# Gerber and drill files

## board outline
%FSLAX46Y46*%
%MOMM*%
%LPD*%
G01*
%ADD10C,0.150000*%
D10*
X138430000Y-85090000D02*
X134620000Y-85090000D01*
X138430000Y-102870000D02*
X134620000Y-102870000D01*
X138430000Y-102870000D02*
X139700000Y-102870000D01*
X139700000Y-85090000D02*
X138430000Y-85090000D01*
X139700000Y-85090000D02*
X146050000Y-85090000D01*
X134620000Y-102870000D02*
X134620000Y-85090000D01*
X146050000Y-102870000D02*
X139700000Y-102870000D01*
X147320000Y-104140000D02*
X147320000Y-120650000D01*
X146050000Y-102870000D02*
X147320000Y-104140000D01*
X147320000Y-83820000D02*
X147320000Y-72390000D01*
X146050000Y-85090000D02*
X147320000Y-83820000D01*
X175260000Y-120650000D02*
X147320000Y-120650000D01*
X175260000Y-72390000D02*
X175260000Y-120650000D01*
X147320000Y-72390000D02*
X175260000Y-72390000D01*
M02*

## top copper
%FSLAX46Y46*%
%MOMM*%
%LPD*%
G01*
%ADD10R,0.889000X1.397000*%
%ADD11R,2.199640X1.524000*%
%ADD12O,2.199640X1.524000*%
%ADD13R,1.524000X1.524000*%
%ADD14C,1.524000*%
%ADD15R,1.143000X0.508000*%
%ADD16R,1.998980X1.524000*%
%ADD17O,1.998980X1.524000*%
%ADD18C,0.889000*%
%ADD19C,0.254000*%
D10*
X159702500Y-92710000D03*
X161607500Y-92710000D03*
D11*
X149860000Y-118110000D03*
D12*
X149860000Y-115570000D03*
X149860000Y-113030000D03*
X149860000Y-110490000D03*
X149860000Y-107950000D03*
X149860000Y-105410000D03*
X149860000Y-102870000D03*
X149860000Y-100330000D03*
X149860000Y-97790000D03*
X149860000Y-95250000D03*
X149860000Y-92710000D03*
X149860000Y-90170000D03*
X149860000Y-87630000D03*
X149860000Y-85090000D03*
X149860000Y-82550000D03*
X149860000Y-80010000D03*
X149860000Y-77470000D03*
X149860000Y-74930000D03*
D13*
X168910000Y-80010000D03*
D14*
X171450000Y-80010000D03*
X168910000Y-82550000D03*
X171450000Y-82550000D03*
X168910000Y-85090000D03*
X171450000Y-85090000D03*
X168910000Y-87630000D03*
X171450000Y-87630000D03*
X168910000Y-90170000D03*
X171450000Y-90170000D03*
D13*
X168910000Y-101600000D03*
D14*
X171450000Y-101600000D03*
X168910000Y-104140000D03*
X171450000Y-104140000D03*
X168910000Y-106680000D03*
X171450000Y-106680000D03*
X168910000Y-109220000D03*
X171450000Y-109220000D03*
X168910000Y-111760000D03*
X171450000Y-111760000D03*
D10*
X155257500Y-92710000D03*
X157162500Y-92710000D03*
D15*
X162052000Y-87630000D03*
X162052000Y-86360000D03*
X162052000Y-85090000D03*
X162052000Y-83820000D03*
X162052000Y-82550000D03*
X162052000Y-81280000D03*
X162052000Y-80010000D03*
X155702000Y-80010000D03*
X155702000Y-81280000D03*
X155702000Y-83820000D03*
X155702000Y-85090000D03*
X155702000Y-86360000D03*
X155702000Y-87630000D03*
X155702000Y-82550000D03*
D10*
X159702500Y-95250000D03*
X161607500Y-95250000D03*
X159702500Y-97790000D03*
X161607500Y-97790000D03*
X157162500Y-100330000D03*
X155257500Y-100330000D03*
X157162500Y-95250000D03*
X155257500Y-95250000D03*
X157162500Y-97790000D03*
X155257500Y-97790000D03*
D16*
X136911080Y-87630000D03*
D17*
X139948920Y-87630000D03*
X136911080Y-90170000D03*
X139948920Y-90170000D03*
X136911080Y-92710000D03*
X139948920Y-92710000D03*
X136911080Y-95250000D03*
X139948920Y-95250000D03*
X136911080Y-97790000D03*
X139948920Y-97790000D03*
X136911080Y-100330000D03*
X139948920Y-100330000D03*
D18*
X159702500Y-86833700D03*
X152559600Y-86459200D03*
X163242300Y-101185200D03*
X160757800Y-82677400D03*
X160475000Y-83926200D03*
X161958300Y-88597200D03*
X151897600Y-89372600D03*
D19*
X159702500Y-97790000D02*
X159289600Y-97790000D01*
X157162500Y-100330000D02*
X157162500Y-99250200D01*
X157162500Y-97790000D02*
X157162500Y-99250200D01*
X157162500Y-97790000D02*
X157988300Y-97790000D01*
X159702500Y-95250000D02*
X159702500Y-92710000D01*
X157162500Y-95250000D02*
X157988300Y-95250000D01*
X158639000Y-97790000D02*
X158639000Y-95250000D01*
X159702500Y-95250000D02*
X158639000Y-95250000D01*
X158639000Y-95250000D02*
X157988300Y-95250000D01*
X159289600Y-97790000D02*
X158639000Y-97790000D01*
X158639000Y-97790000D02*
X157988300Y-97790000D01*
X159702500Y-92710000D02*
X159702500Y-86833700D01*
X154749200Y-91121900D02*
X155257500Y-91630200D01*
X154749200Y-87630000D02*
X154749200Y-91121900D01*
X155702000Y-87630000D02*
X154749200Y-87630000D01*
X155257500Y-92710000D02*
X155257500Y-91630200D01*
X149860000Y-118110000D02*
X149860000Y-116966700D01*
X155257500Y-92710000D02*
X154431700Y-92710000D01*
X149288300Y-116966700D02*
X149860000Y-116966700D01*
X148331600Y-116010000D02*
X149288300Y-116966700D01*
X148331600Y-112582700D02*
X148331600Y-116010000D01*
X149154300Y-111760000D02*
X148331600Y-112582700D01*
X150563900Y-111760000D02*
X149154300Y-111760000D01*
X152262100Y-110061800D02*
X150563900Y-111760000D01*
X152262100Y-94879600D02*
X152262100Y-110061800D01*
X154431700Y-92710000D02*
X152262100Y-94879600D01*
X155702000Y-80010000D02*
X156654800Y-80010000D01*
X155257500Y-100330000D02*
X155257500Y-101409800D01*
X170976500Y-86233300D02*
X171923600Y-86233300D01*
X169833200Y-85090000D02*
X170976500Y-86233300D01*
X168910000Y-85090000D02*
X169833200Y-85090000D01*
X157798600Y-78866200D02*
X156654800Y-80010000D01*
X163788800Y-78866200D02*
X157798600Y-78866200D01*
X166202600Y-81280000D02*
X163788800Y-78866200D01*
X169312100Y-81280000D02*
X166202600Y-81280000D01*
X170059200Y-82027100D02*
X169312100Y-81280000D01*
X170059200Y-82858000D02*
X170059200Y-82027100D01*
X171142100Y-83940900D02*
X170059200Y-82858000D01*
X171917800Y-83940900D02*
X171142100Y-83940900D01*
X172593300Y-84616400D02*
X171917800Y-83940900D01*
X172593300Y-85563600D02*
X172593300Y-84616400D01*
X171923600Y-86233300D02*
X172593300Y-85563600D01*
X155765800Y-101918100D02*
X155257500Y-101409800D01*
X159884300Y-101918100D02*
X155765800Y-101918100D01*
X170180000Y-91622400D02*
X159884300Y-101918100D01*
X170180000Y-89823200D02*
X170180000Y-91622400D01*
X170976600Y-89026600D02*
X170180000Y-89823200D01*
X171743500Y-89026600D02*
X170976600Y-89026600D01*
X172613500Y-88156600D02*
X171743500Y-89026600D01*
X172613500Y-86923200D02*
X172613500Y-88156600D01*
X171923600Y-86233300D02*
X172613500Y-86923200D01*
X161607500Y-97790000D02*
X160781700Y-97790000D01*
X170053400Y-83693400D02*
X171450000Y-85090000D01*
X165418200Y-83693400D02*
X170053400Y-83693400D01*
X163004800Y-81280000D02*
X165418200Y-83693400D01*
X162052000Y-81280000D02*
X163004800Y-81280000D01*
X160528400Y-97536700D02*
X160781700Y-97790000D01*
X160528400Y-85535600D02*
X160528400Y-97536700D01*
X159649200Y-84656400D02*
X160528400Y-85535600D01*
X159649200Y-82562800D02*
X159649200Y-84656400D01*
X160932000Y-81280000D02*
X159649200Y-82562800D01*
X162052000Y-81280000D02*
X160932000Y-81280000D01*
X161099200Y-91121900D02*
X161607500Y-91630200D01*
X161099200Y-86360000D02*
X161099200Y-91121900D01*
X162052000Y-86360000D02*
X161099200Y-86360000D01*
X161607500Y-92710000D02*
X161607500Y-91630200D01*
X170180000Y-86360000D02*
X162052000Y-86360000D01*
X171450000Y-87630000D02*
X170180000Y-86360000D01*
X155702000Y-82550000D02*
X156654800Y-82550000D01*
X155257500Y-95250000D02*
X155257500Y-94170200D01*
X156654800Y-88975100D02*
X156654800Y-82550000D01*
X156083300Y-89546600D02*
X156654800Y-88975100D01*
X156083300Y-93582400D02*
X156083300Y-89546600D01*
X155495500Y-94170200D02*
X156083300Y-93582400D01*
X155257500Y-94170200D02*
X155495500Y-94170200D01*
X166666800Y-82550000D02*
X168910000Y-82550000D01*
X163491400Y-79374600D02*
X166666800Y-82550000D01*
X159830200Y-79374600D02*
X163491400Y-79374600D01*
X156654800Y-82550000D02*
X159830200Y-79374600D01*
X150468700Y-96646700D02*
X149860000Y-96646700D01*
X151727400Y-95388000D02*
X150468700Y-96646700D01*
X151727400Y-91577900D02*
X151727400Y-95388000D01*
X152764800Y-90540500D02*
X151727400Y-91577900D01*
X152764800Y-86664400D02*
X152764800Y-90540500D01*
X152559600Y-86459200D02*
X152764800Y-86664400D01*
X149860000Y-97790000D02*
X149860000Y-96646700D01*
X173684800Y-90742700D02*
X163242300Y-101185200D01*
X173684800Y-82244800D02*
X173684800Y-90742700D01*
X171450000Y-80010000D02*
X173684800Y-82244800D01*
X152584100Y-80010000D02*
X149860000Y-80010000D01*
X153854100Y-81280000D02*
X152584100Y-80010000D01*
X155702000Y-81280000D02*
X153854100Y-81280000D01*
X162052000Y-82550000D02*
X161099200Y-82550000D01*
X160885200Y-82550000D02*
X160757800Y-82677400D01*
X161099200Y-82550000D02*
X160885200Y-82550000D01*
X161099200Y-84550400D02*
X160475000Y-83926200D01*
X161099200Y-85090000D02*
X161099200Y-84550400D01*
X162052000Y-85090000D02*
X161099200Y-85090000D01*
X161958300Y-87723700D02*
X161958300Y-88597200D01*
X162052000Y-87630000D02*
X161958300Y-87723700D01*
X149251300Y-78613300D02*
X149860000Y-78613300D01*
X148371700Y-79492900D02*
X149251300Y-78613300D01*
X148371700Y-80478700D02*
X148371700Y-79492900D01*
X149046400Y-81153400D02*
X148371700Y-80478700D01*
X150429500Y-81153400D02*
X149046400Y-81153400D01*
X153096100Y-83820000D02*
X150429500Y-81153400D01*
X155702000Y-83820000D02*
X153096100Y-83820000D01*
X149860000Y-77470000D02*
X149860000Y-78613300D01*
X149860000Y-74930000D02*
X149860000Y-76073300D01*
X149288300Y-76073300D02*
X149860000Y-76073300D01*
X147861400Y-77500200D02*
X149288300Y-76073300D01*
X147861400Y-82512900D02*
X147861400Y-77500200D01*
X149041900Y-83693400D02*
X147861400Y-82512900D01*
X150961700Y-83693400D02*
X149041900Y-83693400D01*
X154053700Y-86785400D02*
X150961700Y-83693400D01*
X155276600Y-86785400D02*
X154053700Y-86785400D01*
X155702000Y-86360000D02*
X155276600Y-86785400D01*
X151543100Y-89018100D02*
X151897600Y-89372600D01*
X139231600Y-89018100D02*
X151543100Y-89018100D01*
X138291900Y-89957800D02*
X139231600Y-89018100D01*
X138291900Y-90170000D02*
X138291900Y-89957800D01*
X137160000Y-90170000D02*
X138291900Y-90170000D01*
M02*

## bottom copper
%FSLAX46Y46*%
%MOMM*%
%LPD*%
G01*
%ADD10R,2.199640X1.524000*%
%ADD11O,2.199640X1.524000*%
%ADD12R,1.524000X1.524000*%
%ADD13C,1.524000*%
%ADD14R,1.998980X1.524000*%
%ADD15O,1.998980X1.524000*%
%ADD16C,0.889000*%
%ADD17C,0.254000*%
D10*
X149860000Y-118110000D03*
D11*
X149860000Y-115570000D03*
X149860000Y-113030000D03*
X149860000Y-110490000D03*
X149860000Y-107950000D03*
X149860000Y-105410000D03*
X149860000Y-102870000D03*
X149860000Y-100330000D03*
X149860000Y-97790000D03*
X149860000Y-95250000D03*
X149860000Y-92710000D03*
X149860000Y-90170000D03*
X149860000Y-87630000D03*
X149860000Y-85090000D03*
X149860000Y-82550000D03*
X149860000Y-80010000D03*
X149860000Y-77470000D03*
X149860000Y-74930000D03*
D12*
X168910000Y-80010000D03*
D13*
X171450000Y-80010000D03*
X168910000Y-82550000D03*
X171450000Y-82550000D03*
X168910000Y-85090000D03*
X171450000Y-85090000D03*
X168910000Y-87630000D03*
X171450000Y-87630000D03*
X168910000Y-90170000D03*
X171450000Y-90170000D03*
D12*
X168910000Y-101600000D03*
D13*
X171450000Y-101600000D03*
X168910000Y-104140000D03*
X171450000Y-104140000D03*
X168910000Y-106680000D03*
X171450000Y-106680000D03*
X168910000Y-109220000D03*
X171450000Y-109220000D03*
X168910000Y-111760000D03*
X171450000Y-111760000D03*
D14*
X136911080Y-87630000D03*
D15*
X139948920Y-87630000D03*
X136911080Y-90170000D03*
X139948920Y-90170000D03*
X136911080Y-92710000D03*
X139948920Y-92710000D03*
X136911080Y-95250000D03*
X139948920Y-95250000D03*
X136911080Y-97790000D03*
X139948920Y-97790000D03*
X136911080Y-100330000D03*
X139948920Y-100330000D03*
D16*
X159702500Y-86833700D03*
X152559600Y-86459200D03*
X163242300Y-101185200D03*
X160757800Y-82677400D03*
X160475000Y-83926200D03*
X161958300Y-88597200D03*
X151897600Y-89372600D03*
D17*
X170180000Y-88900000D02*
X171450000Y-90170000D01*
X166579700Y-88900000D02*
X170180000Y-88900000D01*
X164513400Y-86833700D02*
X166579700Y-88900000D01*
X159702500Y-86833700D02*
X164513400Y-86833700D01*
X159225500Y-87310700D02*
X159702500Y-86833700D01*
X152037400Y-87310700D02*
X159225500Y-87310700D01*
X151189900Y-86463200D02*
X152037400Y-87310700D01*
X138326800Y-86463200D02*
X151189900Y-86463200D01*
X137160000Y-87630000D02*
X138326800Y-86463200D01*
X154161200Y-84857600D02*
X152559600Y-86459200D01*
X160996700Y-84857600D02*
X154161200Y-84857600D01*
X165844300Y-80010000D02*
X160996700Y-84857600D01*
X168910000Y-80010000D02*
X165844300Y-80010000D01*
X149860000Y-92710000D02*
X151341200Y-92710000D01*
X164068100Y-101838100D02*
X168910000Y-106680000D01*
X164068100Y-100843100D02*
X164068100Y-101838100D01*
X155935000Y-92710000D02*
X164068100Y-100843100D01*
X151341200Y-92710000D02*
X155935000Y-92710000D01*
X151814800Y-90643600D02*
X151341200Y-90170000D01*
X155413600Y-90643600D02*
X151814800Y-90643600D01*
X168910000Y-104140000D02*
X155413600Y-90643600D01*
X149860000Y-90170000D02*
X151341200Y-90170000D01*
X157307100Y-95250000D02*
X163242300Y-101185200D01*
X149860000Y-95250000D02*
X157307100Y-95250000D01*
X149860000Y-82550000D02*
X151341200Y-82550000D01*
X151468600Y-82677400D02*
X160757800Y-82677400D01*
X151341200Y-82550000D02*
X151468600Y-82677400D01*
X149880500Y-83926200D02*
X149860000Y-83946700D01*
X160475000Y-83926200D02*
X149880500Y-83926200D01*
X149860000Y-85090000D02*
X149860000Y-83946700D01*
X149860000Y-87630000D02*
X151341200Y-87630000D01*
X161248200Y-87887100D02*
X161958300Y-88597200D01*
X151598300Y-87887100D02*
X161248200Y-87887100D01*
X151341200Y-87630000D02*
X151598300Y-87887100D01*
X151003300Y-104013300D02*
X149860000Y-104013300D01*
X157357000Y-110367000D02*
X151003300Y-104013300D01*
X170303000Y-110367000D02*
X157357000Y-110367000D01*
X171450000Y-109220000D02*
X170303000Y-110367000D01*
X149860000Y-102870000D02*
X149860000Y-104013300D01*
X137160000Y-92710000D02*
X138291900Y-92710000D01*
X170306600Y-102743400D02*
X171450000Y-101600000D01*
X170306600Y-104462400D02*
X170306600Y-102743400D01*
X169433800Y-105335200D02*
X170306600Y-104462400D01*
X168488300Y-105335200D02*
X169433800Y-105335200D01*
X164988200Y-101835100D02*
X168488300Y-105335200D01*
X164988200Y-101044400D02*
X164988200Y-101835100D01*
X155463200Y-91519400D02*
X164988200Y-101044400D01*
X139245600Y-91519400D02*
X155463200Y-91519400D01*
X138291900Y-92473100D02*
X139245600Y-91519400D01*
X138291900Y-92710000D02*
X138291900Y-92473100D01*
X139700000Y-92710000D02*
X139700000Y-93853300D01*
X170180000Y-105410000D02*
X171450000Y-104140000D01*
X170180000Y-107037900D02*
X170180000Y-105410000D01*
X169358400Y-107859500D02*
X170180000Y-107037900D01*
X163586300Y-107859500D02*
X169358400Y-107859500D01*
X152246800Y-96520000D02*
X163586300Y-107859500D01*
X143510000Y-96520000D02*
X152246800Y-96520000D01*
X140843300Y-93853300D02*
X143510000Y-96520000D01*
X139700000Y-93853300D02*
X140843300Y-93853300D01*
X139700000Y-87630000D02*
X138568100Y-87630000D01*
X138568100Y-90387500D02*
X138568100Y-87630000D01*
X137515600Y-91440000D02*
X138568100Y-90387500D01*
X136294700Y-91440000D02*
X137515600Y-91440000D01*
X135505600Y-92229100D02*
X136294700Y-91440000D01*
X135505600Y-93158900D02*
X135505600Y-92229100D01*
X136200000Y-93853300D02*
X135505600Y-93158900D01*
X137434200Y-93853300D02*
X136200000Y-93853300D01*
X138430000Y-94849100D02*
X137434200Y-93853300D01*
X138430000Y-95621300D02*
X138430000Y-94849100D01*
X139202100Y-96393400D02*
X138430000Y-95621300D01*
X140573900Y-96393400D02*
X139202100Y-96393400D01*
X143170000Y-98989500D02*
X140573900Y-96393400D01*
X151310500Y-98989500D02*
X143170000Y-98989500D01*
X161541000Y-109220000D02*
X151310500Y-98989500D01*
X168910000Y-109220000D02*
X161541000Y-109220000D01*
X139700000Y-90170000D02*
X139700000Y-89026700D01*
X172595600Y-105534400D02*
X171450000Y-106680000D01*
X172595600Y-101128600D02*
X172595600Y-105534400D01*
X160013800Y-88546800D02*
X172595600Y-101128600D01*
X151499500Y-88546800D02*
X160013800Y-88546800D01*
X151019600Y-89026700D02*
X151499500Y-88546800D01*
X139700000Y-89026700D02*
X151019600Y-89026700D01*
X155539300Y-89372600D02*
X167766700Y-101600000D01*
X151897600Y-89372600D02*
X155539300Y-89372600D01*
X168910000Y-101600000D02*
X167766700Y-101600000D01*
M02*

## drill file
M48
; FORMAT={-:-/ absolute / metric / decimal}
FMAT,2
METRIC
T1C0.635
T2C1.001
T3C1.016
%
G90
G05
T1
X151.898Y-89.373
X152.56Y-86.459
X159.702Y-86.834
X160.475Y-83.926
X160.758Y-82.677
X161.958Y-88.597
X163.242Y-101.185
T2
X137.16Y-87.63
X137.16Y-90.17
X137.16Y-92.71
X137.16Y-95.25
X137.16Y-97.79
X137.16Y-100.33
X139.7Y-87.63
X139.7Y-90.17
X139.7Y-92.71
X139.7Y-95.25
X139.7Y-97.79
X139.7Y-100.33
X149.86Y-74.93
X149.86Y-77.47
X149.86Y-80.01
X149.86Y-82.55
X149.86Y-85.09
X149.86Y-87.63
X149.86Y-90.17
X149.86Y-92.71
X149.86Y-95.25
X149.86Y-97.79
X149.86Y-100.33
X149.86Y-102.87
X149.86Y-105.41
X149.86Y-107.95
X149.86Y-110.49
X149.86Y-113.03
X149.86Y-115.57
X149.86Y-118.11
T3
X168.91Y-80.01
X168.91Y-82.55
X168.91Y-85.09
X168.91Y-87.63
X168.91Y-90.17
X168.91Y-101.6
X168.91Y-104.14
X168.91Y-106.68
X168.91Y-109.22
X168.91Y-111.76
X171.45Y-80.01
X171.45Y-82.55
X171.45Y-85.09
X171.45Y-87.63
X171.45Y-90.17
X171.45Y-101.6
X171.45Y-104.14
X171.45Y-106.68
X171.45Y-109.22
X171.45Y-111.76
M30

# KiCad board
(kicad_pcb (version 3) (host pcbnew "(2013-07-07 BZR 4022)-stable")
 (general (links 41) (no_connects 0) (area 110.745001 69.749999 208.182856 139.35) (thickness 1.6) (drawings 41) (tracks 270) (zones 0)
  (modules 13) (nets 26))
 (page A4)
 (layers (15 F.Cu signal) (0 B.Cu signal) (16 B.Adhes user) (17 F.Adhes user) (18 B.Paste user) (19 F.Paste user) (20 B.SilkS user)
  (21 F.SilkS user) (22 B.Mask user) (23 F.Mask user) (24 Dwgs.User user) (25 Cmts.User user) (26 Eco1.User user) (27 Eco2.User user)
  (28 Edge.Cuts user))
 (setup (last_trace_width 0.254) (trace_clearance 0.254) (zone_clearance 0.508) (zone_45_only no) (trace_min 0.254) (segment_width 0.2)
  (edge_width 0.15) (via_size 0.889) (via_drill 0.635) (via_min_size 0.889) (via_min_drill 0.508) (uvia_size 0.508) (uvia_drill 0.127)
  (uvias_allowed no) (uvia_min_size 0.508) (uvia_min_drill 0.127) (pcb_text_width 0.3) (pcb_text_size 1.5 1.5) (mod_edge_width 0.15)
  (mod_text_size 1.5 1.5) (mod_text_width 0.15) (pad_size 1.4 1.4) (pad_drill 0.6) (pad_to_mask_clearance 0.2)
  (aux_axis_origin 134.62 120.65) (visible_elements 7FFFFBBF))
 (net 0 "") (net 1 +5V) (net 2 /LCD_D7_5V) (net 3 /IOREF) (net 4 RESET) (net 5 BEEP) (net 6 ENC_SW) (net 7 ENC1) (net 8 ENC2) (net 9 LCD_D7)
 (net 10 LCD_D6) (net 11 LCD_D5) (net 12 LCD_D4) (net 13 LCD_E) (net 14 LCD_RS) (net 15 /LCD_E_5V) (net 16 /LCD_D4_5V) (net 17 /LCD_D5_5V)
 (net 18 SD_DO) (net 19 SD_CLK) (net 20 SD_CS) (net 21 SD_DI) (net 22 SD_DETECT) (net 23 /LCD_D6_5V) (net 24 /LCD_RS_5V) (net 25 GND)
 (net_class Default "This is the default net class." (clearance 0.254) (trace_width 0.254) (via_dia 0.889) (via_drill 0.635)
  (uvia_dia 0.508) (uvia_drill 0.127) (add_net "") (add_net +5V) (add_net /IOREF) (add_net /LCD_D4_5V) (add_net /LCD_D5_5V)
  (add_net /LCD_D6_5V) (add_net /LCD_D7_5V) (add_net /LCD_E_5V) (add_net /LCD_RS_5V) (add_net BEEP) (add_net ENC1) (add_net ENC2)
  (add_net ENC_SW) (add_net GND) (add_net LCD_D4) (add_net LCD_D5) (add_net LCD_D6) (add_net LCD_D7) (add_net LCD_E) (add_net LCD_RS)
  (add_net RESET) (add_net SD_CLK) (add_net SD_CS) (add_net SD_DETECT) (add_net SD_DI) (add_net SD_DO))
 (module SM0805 (layer F.Cu) (at 160.655 92.71)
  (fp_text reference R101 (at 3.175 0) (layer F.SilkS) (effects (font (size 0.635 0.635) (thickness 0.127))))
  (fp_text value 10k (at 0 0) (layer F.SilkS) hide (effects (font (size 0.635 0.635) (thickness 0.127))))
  (pad 1 smd rect (at -0.9525 0) (size 0.889 1.397) (layers F.Cu F.Paste F.Mask) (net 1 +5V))
  (pad 2 smd rect (at 0.9525 0) (size 0.889 1.397) (layers F.Cu F.Paste F.Mask) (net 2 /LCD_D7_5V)))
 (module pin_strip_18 (layer B.Cu) (at 149.86 96.52 90)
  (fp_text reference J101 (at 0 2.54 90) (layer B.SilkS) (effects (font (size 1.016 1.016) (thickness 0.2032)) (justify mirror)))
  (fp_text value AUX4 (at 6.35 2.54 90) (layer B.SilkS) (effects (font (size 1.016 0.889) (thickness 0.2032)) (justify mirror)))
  (pad 1 thru_hole rect (at -21.59 0 90) (size 1.524 2.19964) (drill 1.00076) (layers *.Cu *.Mask B.SilkS) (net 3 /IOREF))
  (pad 2 thru_hole oval (at -19.05 0 90) (size 1.524 2.19964) (drill 1.00076) (layers *.Cu *.Mask B.SilkS))
  (pad 3 thru_hole oval (at -16.51 0 90) (size 1.524 2.19964) (drill 1.00076) (layers *.Cu *.Mask B.SilkS))
  (pad 4 thru_hole oval (at -13.97 0 90) (size 1.524 2.19964) (drill 1.00076) (layers *.Cu *.Mask B.SilkS))
  (pad 5 thru_hole oval (at -11.43 0 90) (size 1.524 2.19964) (drill 1.00076) (layers *.Cu *.Mask B.SilkS))
  (pad 6 thru_hole oval (at -8.89 0 90) (size 1.524 2.19964) (drill 1.00076) (layers *.Cu *.Mask B.SilkS))
  (pad 7 thru_hole oval (at -6.35 0 90) (size 1.524 2.19964) (drill 1.00076) (layers *.Cu *.Mask B.SilkS) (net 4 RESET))
  (pad 8 thru_hole oval (at -3.81 0 90) (size 1.524 2.19964) (drill 1.00076) (layers *.Cu *.Mask B.SilkS))
  (pad 9 thru_hole oval (at -1.27 0 90) (size 1.524 2.19964) (drill 1.00076) (layers *.Cu *.Mask B.SilkS) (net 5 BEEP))
  (pad 10 thru_hole oval (at 1.27 0 90) (size 1.524 2.19964) (drill 1.00076) (layers *.Cu *.Mask B.SilkS) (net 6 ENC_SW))
  (pad 11 thru_hole oval (at 3.81 0 90) (size 1.524 2.19964) (drill 1.00076) (layers *.Cu *.Mask B.SilkS) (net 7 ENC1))
  (pad 12 thru_hole oval (at 6.35 0 90) (size 1.524 2.19964) (drill 1.00076) (layers *.Cu *.Mask B.SilkS) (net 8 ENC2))
  (pad 13 thru_hole oval (at 8.89 0 90) (size 1.524 2.19964) (drill 1.00076) (layers *.Cu *.Mask B.SilkS) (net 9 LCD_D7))
  (pad 14 thru_hole oval (at 11.43 0 90) (size 1.524 2.19964) (drill 1.00076) (layers *.Cu *.Mask B.SilkS) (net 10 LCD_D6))
  (pad 15 thru_hole oval (at 13.97 0 90) (size 1.524 2.19964) (drill 1.00076) (layers *.Cu *.Mask B.SilkS) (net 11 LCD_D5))
  (pad 16 thru_hole oval (at 16.51 0 90) (size 1.524 2.19964) (drill 1.00076) (layers *.Cu *.Mask B.SilkS) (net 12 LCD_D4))
  (pad 17 thru_hole oval (at 19.05 0 90) (size 1.524 2.19964) (drill 1.00076) (layers *.Cu *.Mask B.SilkS) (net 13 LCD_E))
  (pad 18 thru_hole oval (at 21.59 0 90) (size 1.524 2.19964) (drill 1.00076) (layers *.Cu *.Mask B.SilkS) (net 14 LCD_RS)))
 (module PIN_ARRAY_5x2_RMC (layer F.Cu) (at 170.18 85.09 270)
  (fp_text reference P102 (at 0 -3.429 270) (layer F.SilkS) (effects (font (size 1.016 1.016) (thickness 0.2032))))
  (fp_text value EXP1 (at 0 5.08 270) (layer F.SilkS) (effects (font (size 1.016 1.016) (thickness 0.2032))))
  (pad 1 thru_hole rect (at -5.08 1.27 270) (size 1.524 1.524) (drill 1.016) (layers *.Cu *.Mask F.SilkS) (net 5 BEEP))
  (pad 2 thru_hole circle (at -5.08 -1.27 270) (size 1.524 1.524) (drill 1.016) (layers *.Cu *.Mask F.SilkS) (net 6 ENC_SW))
  (pad 3 thru_hole circle (at -2.54 1.27 270) (size 1.524 1.524) (drill 1.016) (layers *.Cu *.Mask F.SilkS) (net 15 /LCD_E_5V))
  (pad 4 thru_hole circle (at -2.54 -1.27 270) (size 1.524 1.524) (drill 1.016) (layers *.Cu *.Mask F.SilkS))
  (pad 5 thru_hole circle (at 0 1.27 270) (size 1.524 1.524) (drill 1.016) (layers *.Cu *.Mask F.SilkS) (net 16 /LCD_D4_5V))
  (pad 6 thru_hole circle (at 0 -1.27 270) (size 1.524 1.524) (drill 1.016) (layers *.Cu *.Mask F.SilkS) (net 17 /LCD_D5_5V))
  (pad 7 thru_hole circle (at 2.54 1.27 270) (size 1.524 1.524) (drill 1.016) (layers *.Cu *.Mask F.SilkS))
  (pad 8 thru_hole circle (at 2.54 -1.27 270) (size 1.524 1.524) (drill 1.016) (layers *.Cu *.Mask F.SilkS) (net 2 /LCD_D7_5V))
  (pad 9 thru_hole circle (at 5.08 1.27 270) (size 1.524 1.524) (drill 1.016) (layers *.Cu *.Mask F.SilkS))
  (pad 10 thru_hole circle (at 5.08 -1.27 270) (size 1.524 1.524) (drill 1.016) (layers *.Cu *.Mask F.SilkS) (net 1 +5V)))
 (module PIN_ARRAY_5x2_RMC (layer F.Cu) (at 170.18 106.68 270)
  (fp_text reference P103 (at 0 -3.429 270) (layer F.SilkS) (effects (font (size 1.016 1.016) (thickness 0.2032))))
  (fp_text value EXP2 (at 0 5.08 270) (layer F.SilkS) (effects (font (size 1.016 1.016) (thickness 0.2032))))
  (pad 1 thru_hole rect (at -5.08 1.27 270) (size 1.524 1.524) (drill 1.016) (layers *.Cu *.Mask F.SilkS) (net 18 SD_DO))
  (pad 2 thru_hole circle (at -5.08 -1.27 270) (size 1.524 1.524) (drill 1.016) (layers *.Cu *.Mask F.SilkS) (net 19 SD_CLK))
  (pad 3 thru_hole circle (at -2.54 1.27 270) (size 1.524 1.524) (drill 1.016) (layers *.Cu *.Mask F.SilkS) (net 8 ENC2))
  (pad 4 thru_hole circle (at -2.54 -1.27 270) (size 1.524 1.524) (drill 1.016) (layers *.Cu *.Mask F.SilkS) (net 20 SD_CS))
  (pad 5 thru_hole circle (at 0 1.27 270) (size 1.524 1.524) (drill 1.016) (layers *.Cu *.Mask F.SilkS) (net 7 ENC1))
  (pad 6 thru_hole circle (at 0 -1.27 270) (size 1.524 1.524) (drill 1.016) (layers *.Cu *.Mask F.SilkS) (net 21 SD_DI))
  (pad 7 thru_hole circle (at 2.54 1.27 270) (size 1.524 1.524) (drill 1.016) (layers *.Cu *.Mask F.SilkS) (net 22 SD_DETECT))
  (pad 8 thru_hole circle (at 2.54 -1.27 270) (size 1.524 1.524) (drill 1.016) (layers *.Cu *.Mask F.SilkS) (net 4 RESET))
  (pad 9 thru_hole circle (at 5.08 1.27 270) (size 1.524 1.524) (drill 1.016) (layers *.Cu *.Mask F.SilkS))
  (pad 10 thru_hole circle (at 5.08 -1.27 270) (size 1.524 1.524) (drill 1.016) (layers *.Cu *.Mask F.SilkS)))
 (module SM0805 (layer F.Cu) (at 156.21 92.71)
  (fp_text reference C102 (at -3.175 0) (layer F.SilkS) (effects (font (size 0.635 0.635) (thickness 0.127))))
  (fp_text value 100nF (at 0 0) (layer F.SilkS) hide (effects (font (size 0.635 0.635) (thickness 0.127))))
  (pad 1 smd rect (at -0.9525 0) (size 0.889 1.397) (layers F.Cu F.Paste F.Mask) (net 3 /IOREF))
  (pad 2 smd rect (at 0.9525 0) (size 0.889 1.397) (layers F.Cu F.Paste F.Mask)))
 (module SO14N (layer F.Cu) (at 158.75 83.82 90)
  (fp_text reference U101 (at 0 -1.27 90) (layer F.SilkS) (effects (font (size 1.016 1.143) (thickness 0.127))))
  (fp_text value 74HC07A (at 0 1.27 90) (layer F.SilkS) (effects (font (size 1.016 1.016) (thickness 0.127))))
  (pad 1 smd rect (at -3.81 3.302 90) (size 0.508 1.143) (layers F.Cu F.Paste F.Mask) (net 9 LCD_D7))
  (pad 2 smd rect (at -2.54 3.302 90) (size 0.508 1.143) (layers F.Cu F.Paste F.Mask) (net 2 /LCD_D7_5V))
  (pad 3 smd rect (at -1.27 3.302 90) (size 0.508 1.143) (layers F.Cu F.Paste F.Mask) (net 10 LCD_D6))
  (pad 4 smd rect (at 0 3.302 90) (size 0.508 1.143) (layers F.Cu F.Paste F.Mask))
  (pad 5 smd rect (at 1.27 3.302 90) (size 0.508 1.143) (layers F.Cu F.Paste F.Mask) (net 11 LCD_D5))
  (pad 6 smd rect (at 2.54 3.302 90) (size 0.508 1.143) (layers F.Cu F.Paste F.Mask) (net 17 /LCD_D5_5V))
  (pad 7 smd rect (at 3.81 3.302 90) (size 0.508 1.143) (layers F.Cu F.Paste F.Mask))
  (pad 8 smd rect (at 3.81 -3.048 90) (size 0.508 1.143) (layers F.Cu F.Paste F.Mask) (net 16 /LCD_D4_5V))
  (pad 9 smd rect (at 2.54 -3.048 90) (size 0.508 1.143) (layers F.Cu F.Paste F.Mask) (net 12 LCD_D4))
  (pad 11 smd rect (at 0 -3.048 90) (size 0.508 1.143) (layers F.Cu F.Paste F.Mask) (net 13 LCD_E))
  (pad 12 smd rect (at -1.27 -3.048 90) (size 0.508 1.143) (layers F.Cu F.Paste F.Mask))
  (pad 13 smd rect (at -2.54 -3.048 90) (size 0.508 1.143) (layers F.Cu F.Paste F.Mask) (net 14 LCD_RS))
  (pad 14 smd rect (at -3.81 -3.048 90) (size 0.508 1.143) (layers F.Cu F.Paste F.Mask) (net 3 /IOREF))
  (pad 10 smd rect (at 1.27 -3.048 90) (size 0.508 1.143) (layers F.Cu F.Paste F.Mask) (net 15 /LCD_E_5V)))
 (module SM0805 (layer F.Cu) (at 160.655 95.25)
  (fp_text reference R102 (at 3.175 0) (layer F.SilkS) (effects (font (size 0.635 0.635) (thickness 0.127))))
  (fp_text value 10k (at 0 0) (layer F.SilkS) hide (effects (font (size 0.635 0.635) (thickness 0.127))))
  (pad 1 smd rect (at -0.9525 0) (size 0.889 1.397) (layers F.Cu F.Paste F.Mask) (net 1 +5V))
  (pad 2 smd rect (at 0.9525 0) (size 0.889 1.397) (layers F.Cu F.Paste F.Mask)))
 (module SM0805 (layer F.Cu) (at 160.655 97.79)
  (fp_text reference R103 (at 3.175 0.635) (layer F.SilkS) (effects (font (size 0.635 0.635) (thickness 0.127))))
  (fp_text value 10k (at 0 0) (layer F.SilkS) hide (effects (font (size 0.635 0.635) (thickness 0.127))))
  (pad 1 smd rect (at -0.9525 0) (size 0.889 1.397) (layers F.Cu F.Paste F.Mask) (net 1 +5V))
  (pad 2 smd rect (at 0.9525 0) (size 0.889 1.397) (layers F.Cu F.Paste F.Mask) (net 17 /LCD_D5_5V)))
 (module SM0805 (layer F.Cu) (at 156.21 100.33 180)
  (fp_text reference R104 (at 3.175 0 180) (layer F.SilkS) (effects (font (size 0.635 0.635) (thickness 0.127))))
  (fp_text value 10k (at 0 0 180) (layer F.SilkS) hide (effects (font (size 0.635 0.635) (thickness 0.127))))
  (pad 1 smd rect (at -0.9525 0 180) (size 0.889 1.397) (layers F.Cu F.Paste F.Mask) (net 1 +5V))
  (pad 2 smd rect (at 0.9525 0 180) (size 0.889 1.397) (layers F.Cu F.Paste F.Mask) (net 16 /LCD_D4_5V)))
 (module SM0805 (layer F.Cu) (at 156.21 95.25 180)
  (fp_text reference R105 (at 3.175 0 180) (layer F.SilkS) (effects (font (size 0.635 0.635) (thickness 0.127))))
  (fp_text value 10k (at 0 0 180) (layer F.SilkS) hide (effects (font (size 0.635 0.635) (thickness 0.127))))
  (pad 1 smd rect (at -0.9525 0 180) (size 0.889 1.397) (layers F.Cu F.Paste F.Mask) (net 1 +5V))
  (pad 2 smd rect (at 0.9525 0 180) (size 0.889 1.397) (layers F.Cu F.Paste F.Mask) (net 15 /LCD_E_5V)))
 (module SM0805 (layer F.Cu) (at 156.21 97.79 180)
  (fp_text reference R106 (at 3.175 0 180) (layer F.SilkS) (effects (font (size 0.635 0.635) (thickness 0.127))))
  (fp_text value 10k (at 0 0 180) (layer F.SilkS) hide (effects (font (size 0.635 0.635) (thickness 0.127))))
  (pad 1 smd rect (at -0.9525 0 180) (size 0.889 1.397) (layers F.Cu F.Paste F.Mask) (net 1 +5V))
  (pad 2 smd rect (at 0.9525 0 180) (size 0.889 1.397) (layers F.Cu F.Paste F.Mask)))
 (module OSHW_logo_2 (layer F.Cu) (at 158.75 110.49)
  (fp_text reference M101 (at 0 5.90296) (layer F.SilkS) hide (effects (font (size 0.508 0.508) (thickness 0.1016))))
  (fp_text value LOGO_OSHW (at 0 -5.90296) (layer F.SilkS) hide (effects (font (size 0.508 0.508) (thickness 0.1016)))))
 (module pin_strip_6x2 (layer F.Cu) (at 138.43 93.98 270)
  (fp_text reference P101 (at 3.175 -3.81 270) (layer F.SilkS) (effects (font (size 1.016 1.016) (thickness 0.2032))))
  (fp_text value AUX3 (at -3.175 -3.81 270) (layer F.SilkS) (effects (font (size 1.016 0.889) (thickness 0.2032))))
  (pad 1 thru_hole rect (at -6.35 1.27 270) (size 1.524 1.99898) (drill 1.00076 (offset 0 0.24892)) (layers *.Cu *.Mask F.SilkS) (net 1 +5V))
  (pad 2 thru_hole oval (at -6.35 -1.27 270) (size 1.524 1.99898) (drill 1.00076 (offset 0 -0.24892)) (layers *.Cu *.Mask F.SilkS)
   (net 22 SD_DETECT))
  (pad 3 thru_hole oval (at -3.81 1.27 270) (size 1.524 1.99898) (drill 1.00076 (offset 0 0.24892)) (layers *.Cu *.Mask F.SilkS)
   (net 18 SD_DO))
  (pad 4 thru_hole oval (at -3.81 -1.27 270) (size 1.524 1.99898) (drill 1.00076 (offset 0 -0.24892)) (layers *.Cu *.Mask F.SilkS)
   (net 21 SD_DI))
  (pad 5 thru_hole oval (at -1.27 1.27 270) (size 1.524 1.99898) (drill 1.00076 (offset 0 0.24892)) (layers *.Cu *.Mask F.SilkS)
   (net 19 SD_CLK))
  (pad 6 thru_hole oval (at -1.27 -1.27 270) (size 1.524 1.99898) (drill 1.00076 (offset 0 -0.24892)) (layers *.Cu *.Mask F.SilkS)
   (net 20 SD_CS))
  (pad 7 thru_hole oval (at 1.27 1.27 270) (size 1.524 1.99898) (drill 1.00076 (offset 0 0.24892)) (layers *.Cu *.Mask F.SilkS))
  (pad 8 thru_hole oval (at 1.27 -1.27 270) (size 1.524 1.99898) (drill 1.00076 (offset 0 -0.24892)) (layers *.Cu *.Mask F.SilkS))
  (pad 9 thru_hole oval (at 3.81 1.27 270) (size 1.524 1.99898) (drill 1.00076 (offset 0 0.24892)) (layers *.Cu *.Mask F.SilkS))
  (pad 10 thru_hole oval (at 3.81 -1.27 270) (size 1.524 1.99898) (drill 1.00076 (offset 0 -0.24892)) (layers *.Cu *.Mask F.SilkS))
  (pad 11 thru_hole oval (at 6.35 1.27 270) (size 1.524 1.99898) (drill 1.00076 (offset 0 0.24892)) (layers *.Cu *.Mask F.SilkS))
  (pad 12 thru_hole oval (at 6.35 -1.27 270) (size 1.524 1.99898) (drill 1.00076 (offset 0 -0.24892)) (layers *.Cu *.Mask F.SilkS)))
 (gr_line (start 138.43 85.09) (end 134.62 85.09) (angle 90) (layer Edge.Cuts) (width 0.15))
 (gr_line (start 138.43 102.87) (end 134.62 102.87) (angle 90) (layer Edge.Cuts) (width 0.15))
 (gr_line (start 138.43 102.87) (end 139.7 102.87) (angle 90) (layer Edge.Cuts) (width 0.15))
 (gr_line (start 139.7 85.09) (end 138.43 85.09) (angle 90) (layer Edge.Cuts) (width 0.15))
 (gr_line (start 139.7 85.09) (end 146.05 85.09) (angle 90) (layer Edge.Cuts) (width 0.15))
 (gr_line (start 134.62 102.87) (end 134.62 85.09) (angle 90) (layer Edge.Cuts) (width 0.15))
 (gr_line (start 146.05 102.87) (end 139.7 102.87) (angle 90) (layer Edge.Cuts) (width 0.15))
 (gr_line (start 147.32 104.14) (end 147.32 120.65) (angle 90) (layer Edge.Cuts) (width 0.15))
 (gr_line (start 146.05 102.87) (end 147.32 104.14) (angle 90) (layer Edge.Cuts) (width 0.15))
 (gr_line (start 147.32 83.82) (end 147.32 72.39) (angle 90) (layer Edge.Cuts) (width 0.15))
 (gr_line (start 146.05 85.09) (end 147.32 83.82) (angle 90) (layer Edge.Cuts) (width 0.15))
 (gr_line (start 175.26 120.65) (end 147.32 120.65) (angle 90) (layer Edge.Cuts) (width 0.15))
 (gr_line (start 175.26 72.39) (end 175.26 120.65) (angle 90) (layer Edge.Cuts) (width 0.15))
 (gr_line (start 147.32 72.39) (end 175.26 72.39) (angle 90) (layer Edge.Cuts) (width 0.15))
 (via (at 159.7025 86.8337) (size 0.889) (layers F.Cu B.Cu) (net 1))
 (via (at 152.5596 86.4592) (size 0.889) (layers F.Cu B.Cu) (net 5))
 (via (at 163.2423 101.1852) (size 0.889) (layers F.Cu B.Cu) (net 6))
 (via (at 160.7578 82.6774) (size 0.889) (layers F.Cu B.Cu) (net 11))
 (via (at 160.475 83.9262) (size 0.889) (layers F.Cu B.Cu) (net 10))
 (via (at 161.9583 88.5972) (size 0.889) (layers F.Cu B.Cu) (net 9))
 (via (at 151.8976 89.3726) (size 0.889) (layers F.Cu B.Cu) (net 18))
 (segment (start 159.7025 97.79) (end 159.2896 97.79) (width 0.254) (layer F.Cu) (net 1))
 (segment (start 157.1625 100.33) (end 157.1625 99.2502) (width 0.254) (layer F.Cu) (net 1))
 (segment (start 157.1625 97.79) (end 157.1625 99.2502) (width 0.254) (layer F.Cu) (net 1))
 (segment (start 157.1625 97.79) (end 157.9883 97.79) (width 0.254) (layer F.Cu) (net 1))
 (segment (start 159.7025 95.25) (end 159.7025 92.71) (width 0.254) (layer F.Cu) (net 1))
 (segment (start 157.1625 95.25) (end 157.9883 95.25) (width 0.254) (layer F.Cu) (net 1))
 (segment (start 158.639 97.79) (end 158.639 95.25) (width 0.254) (layer F.Cu) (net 1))
 (segment (start 159.7025 95.25) (end 158.639 95.25) (width 0.254) (layer F.Cu) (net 1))
 (segment (start 158.639 95.25) (end 157.9883 95.25) (width 0.254) (layer F.Cu) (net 1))
 (segment (start 159.2896 97.79) (end 158.639 97.79) (width 0.254) (layer F.Cu) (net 1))
 (segment (start 158.639 97.79) (end 157.9883 97.79) (width 0.254) (layer F.Cu) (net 1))
 (segment (start 159.7025 92.71) (end 159.7025 86.8337) (width 0.254) (layer F.Cu) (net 1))
 (segment (start 170.18 88.9) (end 171.45 90.17) (width 0.254) (layer B.Cu) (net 1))
 (segment (start 166.5797 88.9) (end 170.18 88.9) (width 0.254) (layer B.Cu) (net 1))
 (segment (start 164.5134 86.8337) (end 166.5797 88.9) (width 0.254) (layer B.Cu) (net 1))
 (segment (start 159.7025 86.8337) (end 164.5134 86.8337) (width 0.254) (layer B.Cu) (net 1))
 (segment (start 159.2255 87.3107) (end 159.7025 86.8337) (width 0.254) (layer B.Cu) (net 1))
 (segment (start 152.0374 87.3107) (end 159.2255 87.3107) (width 0.254) (layer B.Cu) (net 1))
 (segment (start 151.1899 86.4632) (end 152.0374 87.3107) (width 0.254) (layer B.Cu) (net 1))
 (segment (start 138.3268 86.4632) (end 151.1899 86.4632) (width 0.254) (layer B.Cu) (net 1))
 (segment (start 137.16 87.63) (end 138.3268 86.4632) (width 0.254) (layer B.Cu) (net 1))
 (segment (start 154.7492 91.1219) (end 155.2575 91.6302) (width 0.254) (layer F.Cu) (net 3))
 (segment (start 154.7492 87.63) (end 154.7492 91.1219) (width 0.254) (layer F.Cu) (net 3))
 (segment (start 155.702 87.63) (end 154.7492 87.63) (width 0.254) (layer F.Cu) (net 3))
 (segment (start 155.2575 92.71) (end 155.2575 91.6302) (width 0.254) (layer F.Cu) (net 3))
 (segment (start 149.86 118.11) (end 149.86 116.9667) (width 0.254) (layer F.Cu) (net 3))
 (segment (start 155.2575 92.71) (end 154.4317 92.71) (width 0.254) (layer F.Cu) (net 3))
 (segment (start 149.2883 116.9667) (end 149.86 116.9667) (width 0.254) (layer F.Cu) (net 3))
 (segment (start 148.3316 116.01) (end 149.2883 116.9667) (width 0.254) (layer F.Cu) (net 3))
 (segment (start 148.3316 112.5827) (end 148.3316 116.01) (width 0.254) (layer F.Cu) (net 3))
 (segment (start 149.1543 111.76) (end 148.3316 112.5827) (width 0.254) (layer F.Cu) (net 3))
 (segment (start 150.5639 111.76) (end 149.1543 111.76) (width 0.254) (layer F.Cu) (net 3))
 (segment (start 152.2621 110.0618) (end 150.5639 111.76) (width 0.254) (layer F.Cu) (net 3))
 (segment (start 152.2621 94.8796) (end 152.2621 110.0618) (width 0.254) (layer F.Cu) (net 3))
 (segment (start 154.4317 92.71) (end 152.2621 94.8796) (width 0.254) (layer F.Cu) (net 3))
 (segment (start 155.702 80.01) (end 156.6548 80.01) (width 0.254) (layer F.Cu) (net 16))
 (segment (start 155.2575 100.33) (end 155.2575 101.4098) (width 0.254) (layer F.Cu) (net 16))
 (segment (start 170.9765 86.2333) (end 171.9236 86.2333) (width 0.254) (layer F.Cu) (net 16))
 (segment (start 169.8332 85.09) (end 170.9765 86.2333) (width 0.254) (layer F.Cu) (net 16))
 (segment (start 168.91 85.09) (end 169.8332 85.09) (width 0.254) (layer F.Cu) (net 16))
 (segment (start 157.7986 78.8662) (end 156.6548 80.01) (width 0.254) (layer F.Cu) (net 16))
 (segment (start 163.7888 78.8662) (end 157.7986 78.8662) (width 0.254) (layer F.Cu) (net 16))
 (segment (start 166.2026 81.28) (end 163.7888 78.8662) (width 0.254) (layer F.Cu) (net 16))
 (segment (start 169.3121 81.28) (end 166.2026 81.28) (width 0.254) (layer F.Cu) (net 16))
 (segment (start 170.0592 82.0271) (end 169.3121 81.28) (width 0.254) (layer F.Cu) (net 16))
 (segment (start 170.0592 82.858) (end 170.0592 82.0271) (width 0.254) (layer F.Cu) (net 16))
 (segment (start 171.1421 83.9409) (end 170.0592 82.858) (width 0.254) (layer F.Cu) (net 16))
 (segment (start 171.9178 83.9409) (end 171.1421 83.9409) (width 0.254) (layer F.Cu) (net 16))
 (segment (start 172.5933 84.6164) (end 171.9178 83.9409) (width 0.254) (layer F.Cu) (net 16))
 (segment (start 172.5933 85.5636) (end 172.5933 84.6164) (width 0.254) (layer F.Cu) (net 16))
 (segment (start 171.9236 86.2333) (end 172.5933 85.5636) (width 0.254) (layer F.Cu) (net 16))
 (segment (start 155.7658 101.9181) (end 155.2575 101.4098) (width 0.254) (layer F.Cu) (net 16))
 (segment (start 159.8843 101.9181) (end 155.7658 101.9181) (width 0.254) (layer F.Cu) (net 16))
 (segment (start 170.18 91.6224) (end 159.8843 101.9181) (width 0.254) (layer F.Cu) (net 16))
 (segment (start 170.18 89.8232) (end 170.18 91.6224) (width 0.254) (layer F.Cu) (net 16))
 (segment (start 170.9766 89.0266) (end 170.18 89.8232) (width 0.254) (layer F.Cu) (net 16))
 (segment (start 171.7435 89.0266) (end 170.9766 89.0266) (width 0.254) (layer F.Cu) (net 16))
 (segment (start 172.6135 88.1566) (end 171.7435 89.0266) (width 0.254) (layer F.Cu) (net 16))
 (segment (start 172.6135 86.9232) (end 172.6135 88.1566) (width 0.254) (layer F.Cu) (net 16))
 (segment (start 171.9236 86.2333) (end 172.6135 86.9232) (width 0.254) (layer F.Cu) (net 16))
 (segment (start 161.6075 97.79) (end 160.7817 97.79) (width 0.254) (layer F.Cu) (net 17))
 (segment (start 170.0534 83.6934) (end 171.45 85.09) (width 0.254) (layer F.Cu) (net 17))
 (segment (start 165.4182 83.6934) (end 170.0534 83.6934) (width 0.254) (layer F.Cu) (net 17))
 (segment (start 163.0048 81.28) (end 165.4182 83.6934) (width 0.254) (layer F.Cu) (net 17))
 (segment (start 162.052 81.28) (end 163.0048 81.28) (width 0.254) (layer F.Cu) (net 17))
 (segment (start 160.5284 97.5367) (end 160.7817 97.79) (width 0.254) (layer F.Cu) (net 17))
 (segment (start 160.5284 85.5356) (end 160.5284 97.5367) (width 0.254) (layer F.Cu) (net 17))
 (segment (start 159.6492 84.6564) (end 160.5284 85.5356) (width 0.254) (layer F.Cu) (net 17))
 (segment (start 159.6492 82.5628) (end 159.6492 84.6564) (width 0.254) (layer F.Cu) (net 17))
 (segment (start 160.932 81.28) (end 159.6492 82.5628) (width 0.254) (layer F.Cu) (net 17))
 (segment (start 162.052 81.28) (end 160.932 81.28) (width 0.254) (layer F.Cu) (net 17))
 (segment (start 161.0992 91.1219) (end 161.6075 91.6302) (width 0.254) (layer F.Cu) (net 2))
 (segment (start 161.0992 86.36) (end 161.0992 91.1219) (width 0.254) (layer F.Cu) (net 2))
 (segment (start 162.052 86.36) (end 161.0992 86.36) (width 0.254) (layer F.Cu) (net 2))
 (segment (start 161.6075 92.71) (end 161.6075 91.6302) (width 0.254) (layer F.Cu) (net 2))
 (segment (start 170.18 86.36) (end 162.052 86.36) (width 0.254) (layer F.Cu) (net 2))
 (segment (start 171.45 87.63) (end 170.18 86.36) (width 0.254) (layer F.Cu) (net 2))
 (segment (start 155.702 82.55) (end 156.6548 82.55) (width 0.254) (layer F.Cu) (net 15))
 (segment (start 155.2575 95.25) (end 155.2575 94.1702) (width 0.254) (layer F.Cu) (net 15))
 (segment (start 156.6548 88.9751) (end 156.6548 82.55) (width 0.254) (layer F.Cu) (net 15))
 (segment (start 156.0833 89.5466) (end 156.6548 88.9751) (width 0.254) (layer F.Cu) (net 15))
 (segment (start 156.0833 93.5824) (end 156.0833 89.5466) (width 0.254) (layer F.Cu) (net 15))
 (segment (start 155.4955 94.1702) (end 156.0833 93.5824) (width 0.254) (layer F.Cu) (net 15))
 (segment (start 155.2575 94.1702) (end 155.4955 94.1702) (width 0.254) (layer F.Cu) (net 15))
 (segment (start 166.6668 82.55) (end 168.91 82.55) (width 0.254) (layer F.Cu) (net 15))
 (segment (start 163.4914 79.3746) (end 166.6668 82.55) (width 0.254) (layer F.Cu) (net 15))
 (segment (start 159.8302 79.3746) (end 163.4914 79.3746) (width 0.254) (layer F.Cu) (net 15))
 (segment (start 156.6548 82.55) (end 159.8302 79.3746) (width 0.254) (layer F.Cu) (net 15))
 (segment (start 154.1612 84.8576) (end 152.5596 86.4592) (width 0.254) (layer B.Cu) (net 5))
 (segment (start 160.9967 84.8576) (end 154.1612 84.8576) (width 0.254) (layer B.Cu) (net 5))
 (segment (start 165.8443 80.01) (end 160.9967 84.8576) (width 0.254) (layer B.Cu) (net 5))
 (segment (start 168.91 80.01) (end 165.8443 80.01) (width 0.254) (layer B.Cu) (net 5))
 (segment (start 150.4687 96.6467) (end 149.86 96.6467) (width 0.254) (layer F.Cu) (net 5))
 (segment (start 151.7274 95.388) (end 150.4687 96.6467) (width 0.254) (layer F.Cu) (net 5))
 (segment (start 151.7274 91.5779) (end 151.7274 95.388) (width 0.254) (layer F.Cu) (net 5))
 (segment (start 152.7648 90.5405) (end 151.7274 91.5779) (width 0.254) (layer F.Cu) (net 5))
 (segment (start 152.7648 86.6644) (end 152.7648 90.5405) (width 0.254) (layer F.Cu) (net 5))
 (segment (start 152.5596 86.4592) (end 152.7648 86.6644) (width 0.254) (layer F.Cu) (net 5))
 (segment (start 149.86 97.79) (end 149.86 96.6467) (width 0.254) (layer F.Cu) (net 5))
 (segment (start 149.86 92.71) (end 151.3412 92.71) (width 0.254) (layer B.Cu) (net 7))
 (segment (start 164.0681 101.8381) (end 168.91 106.68) (width 0.254) (layer B.Cu) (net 7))
 (segment (start 164.0681 100.8431) (end 164.0681 101.8381) (width 0.254) (layer B.Cu) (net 7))
 (segment (start 155.935 92.71) (end 164.0681 100.8431) (width 0.254) (layer B.Cu) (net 7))
 (segment (start 151.3412 92.71) (end 155.935 92.71) (width 0.254) (layer B.Cu) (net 7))
 (segment (start 151.8148 90.6436) (end 151.3412 90.17) (width 0.254) (layer B.Cu) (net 8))
 (segment (start 155.4136 90.6436) (end 151.8148 90.6436) (width 0.254) (layer B.Cu) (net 8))
 (segment (start 168.91 104.14) (end 155.4136 90.6436) (width 0.254) (layer B.Cu) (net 8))
 (segment (start 149.86 90.17) (end 151.3412 90.17) (width 0.254) (layer B.Cu) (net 8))
 (segment (start 173.6848 90.7427) (end 163.2423 101.1852) (width 0.254) (layer F.Cu) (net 6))
 (segment (start 173.6848 82.2448) (end 173.6848 90.7427) (width 0.254) (layer F.Cu) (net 6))
 (segment (start 171.45 80.01) (end 173.6848 82.2448) (width 0.254) (layer F.Cu) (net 6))
 (segment (start 157.3071 95.25) (end 163.2423 101.1852) (width 0.254) (layer B.Cu) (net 6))
 (segment (start 149.86 95.25) (end 157.3071 95.25) (width 0.254) (layer B.Cu) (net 6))
 (segment (start 152.5841 80.01) (end 149.86 80.01) (width 0.254) (layer F.Cu) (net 12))
 (segment (start 153.8541 81.28) (end 152.5841 80.01) (width 0.254) (layer F.Cu) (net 12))
 (segment (start 155.702 81.28) (end 153.8541 81.28) (width 0.254) (layer F.Cu) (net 12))
 (segment (start 162.052 82.55) (end 161.0992 82.55) (width 0.254) (layer F.Cu) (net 11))
 (segment (start 160.8852 82.55) (end 160.7578 82.6774) (width 0.254) (layer F.Cu) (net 11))
 (segment (start 161.0992 82.55) (end 160.8852 82.55) (width 0.254) (layer F.Cu) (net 11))
 (segment (start 149.86 82.55) (end 151.3412 82.55) (width 0.254) (layer B.Cu) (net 11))
 (segment (start 151.4686 82.6774) (end 160.7578 82.6774) (width 0.254) (layer B.Cu) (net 11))
 (segment (start 151.3412 82.55) (end 151.4686 82.6774) (width 0.254) (layer B.Cu) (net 11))
 (segment (start 161.0992 84.5504) (end 160.475 83.9262) (width 0.254) (layer F.Cu) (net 10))
 (segment (start 161.0992 85.09) (end 161.0992 84.5504) (width 0.254) (layer F.Cu) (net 10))
 (segment (start 149.8805 83.9262) (end 149.86 83.9467) (width 0.254) (layer B.Cu) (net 10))
 (segment (start 160.475 83.9262) (end 149.8805 83.9262) (width 0.254) (layer B.Cu) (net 10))
 (segment (start 162.052 85.09) (end 161.0992 85.09) (width 0.254) (layer F.Cu) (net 10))
 (segment (start 149.86 85.09) (end 149.86 83.9467) (width 0.254) (layer B.Cu) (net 10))
 (segment (start 149.86 87.63) (end 151.3412 87.63) (width 0.254) (layer B.Cu) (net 9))
 (segment (start 161.9583 87.7237) (end 161.9583 88.5972) (width 0.254) (layer F.Cu) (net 9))
 (segment (start 162.052 87.63) (end 161.9583 87.7237) (width 0.254) (layer F.Cu) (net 9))
 (segment (start 161.2482 87.8871) (end 161.9583 88.5972) (width 0.254) (layer B.Cu) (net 9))
 (segment (start 151.5983 87.8871) (end 161.2482 87.8871) (width 0.254) (layer B.Cu) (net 9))
 (segment (start 151.3412 87.63) (end 151.5983 87.8871) (width 0.254) (layer B.Cu) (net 9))
 (segment (start 149.2513 78.6133) (end 149.86 78.6133) (width 0.254) (layer F.Cu) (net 13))
 (segment (start 148.3717 79.4929) (end 149.2513 78.6133) (width 0.254) (layer F.Cu) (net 13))
 (segment (start 148.3717 80.4787) (end 148.3717 79.4929) (width 0.254) (layer F.Cu) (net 13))
 (segment (start 149.0464 81.1534) (end 148.3717 80.4787) (width 0.254) (layer F.Cu) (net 13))
 (segment (start 150.4295 81.1534) (end 149.0464 81.1534) (width 0.254) (layer F.Cu) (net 13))
 (segment (start 153.0961 83.82) (end 150.4295 81.1534) (width 0.254) (layer F.Cu) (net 13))
 (segment (start 155.702 83.82) (end 153.0961 83.82) (width 0.254) (layer F.Cu) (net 13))
 (segment (start 149.86 77.47) (end 149.86 78.6133) (width 0.254) (layer F.Cu) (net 13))
 (segment (start 149.86 74.93) (end 149.86 76.0733) (width 0.254) (layer F.Cu) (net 14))
 (segment (start 149.2883 76.0733) (end 149.86 76.0733) (width 0.254) (layer F.Cu) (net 14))
 (segment (start 147.8614 77.5002) (end 149.2883 76.0733) (width 0.254) (layer F.Cu) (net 14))
 (segment (start 147.8614 82.5129) (end 147.8614 77.5002) (width 0.254) (layer F.Cu) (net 14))
 (segment (start 149.0419 83.6934) (end 147.8614 82.5129) (width 0.254) (layer F.Cu) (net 14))
 (segment (start 150.9617 83.6934) (end 149.0419 83.6934) (width 0.254) (layer F.Cu) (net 14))
 (segment (start 154.0537 86.7854) (end 150.9617 83.6934) (width 0.254) (layer F.Cu) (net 14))
 (segment (start 155.2766 86.7854) (end 154.0537 86.7854) (width 0.254) (layer F.Cu) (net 14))
 (segment (start 155.702 86.36) (end 155.2766 86.7854) (width 0.254) (layer F.Cu) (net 14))
 (segment (start 151.0033 104.0133) (end 149.86 104.0133) (width 0.254) (layer B.Cu) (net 4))
 (segment (start 157.357 110.367) (end 151.0033 104.0133) (width 0.254) (layer B.Cu) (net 4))
 (segment (start 170.303 110.367) (end 157.357 110.367) (width 0.254) (layer B.Cu) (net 4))
 (segment (start 171.45 109.22) (end 170.303 110.367) (width 0.254) (layer B.Cu) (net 4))
 (segment (start 149.86 102.87) (end 149.86 104.0133) (width 0.254) (layer B.Cu) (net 4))
 (segment (start 137.16 92.71) (end 138.2919 92.71) (width 0.254) (layer B.Cu) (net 19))
 (segment (start 170.3066 102.7434) (end 171.45 101.6) (width 0.254) (layer B.Cu) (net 19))
 (segment (start 170.3066 104.4624) (end 170.3066 102.7434) (width 0.254) (layer B.Cu) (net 19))
 (segment (start 169.4338 105.3352) (end 170.3066 104.4624) (width 0.254) (layer B.Cu) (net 19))
 (segment (start 168.4883 105.3352) (end 169.4338 105.3352) (width 0.254) (layer B.Cu) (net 19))
 (segment (start 164.9882 101.8351) (end 168.4883 105.3352) (width 0.254) (layer B.Cu) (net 19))
 (segment (start 164.9882 101.0444) (end 164.9882 101.8351) (width 0.254) (layer B.Cu) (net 19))
 (segment (start 155.4632 91.5194) (end 164.9882 101.0444) (width 0.254) (layer B.Cu) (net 19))
 (segment (start 139.2456 91.5194) (end 155.4632 91.5194) (width 0.254) (layer B.Cu) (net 19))
 (segment (start 138.2919 92.4731) (end 139.2456 91.5194) (width 0.254) (layer B.Cu) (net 19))
 (segment (start 138.2919 92.71) (end 138.2919 92.4731) (width 0.254) (layer B.Cu) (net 19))
 (segment (start 139.7 92.71) (end 139.7 93.8533) (width 0.254) (layer B.Cu) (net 20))
 (segment (start 170.18 105.41) (end 171.45 104.14) (width 0.254) (layer B.Cu) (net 20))
 (segment (start 170.18 107.0379) (end 170.18 105.41) (width 0.254) (layer B.Cu) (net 20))
 (segment (start 169.3584 107.8595) (end 170.18 107.0379) (width 0.254) (layer B.Cu) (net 20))
 (segment (start 163.5863 107.8595) (end 169.3584 107.8595) (width 0.254) (layer B.Cu) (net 20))
 (segment (start 152.2468 96.52) (end 163.5863 107.8595) (width 0.254) (layer B.Cu) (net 20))
 (segment (start 143.51 96.52) (end 152.2468 96.52) (width 0.254) (layer B.Cu) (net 20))
 (segment (start 140.8433 93.8533) (end 143.51 96.52) (width 0.254) (layer B.Cu) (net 20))
 (segment (start 139.7 93.8533) (end 140.8433 93.8533) (width 0.254) (layer B.Cu) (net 20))
 (segment (start 139.7 87.63) (end 138.5681 87.63) (width 0.254) (layer B.Cu) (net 22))
 (segment (start 138.5681 90.3875) (end 138.5681 87.63) (width 0.254) (layer B.Cu) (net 22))
 (segment (start 137.5156 91.44) (end 138.5681 90.3875) (width 0.254) (layer B.Cu) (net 22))
 (segment (start 136.2947 91.44) (end 137.5156 91.44) (width 0.254) (layer B.Cu) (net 22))
 (segment (start 135.5056 92.2291) (end 136.2947 91.44) (width 0.254) (layer B.Cu) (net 22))
 (segment (start 135.5056 93.1589) (end 135.5056 92.2291) (width 0.254) (layer B.Cu) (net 22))
 (segment (start 136.2 93.8533) (end 135.5056 93.1589) (width 0.254) (layer B.Cu) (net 22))
 (segment (start 137.4342 93.8533) (end 136.2 93.8533) (width 0.254) (layer B.Cu) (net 22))
 (segment (start 138.43 94.8491) (end 137.4342 93.8533) (width 0.254) (layer B.Cu) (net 22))
 (segment (start 138.43 95.6213) (end 138.43 94.8491) (width 0.254) (layer B.Cu) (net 22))
 (segment (start 139.2021 96.3934) (end 138.43 95.6213) (width 0.254) (layer B.Cu) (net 22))
 (segment (start 140.5739 96.3934) (end 139.2021 96.3934) (width 0.254) (layer B.Cu) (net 22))
 (segment (start 143.17 98.9895) (end 140.5739 96.3934) (width 0.254) (layer B.Cu) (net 22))
 (segment (start 151.3105 98.9895) (end 143.17 98.9895) (width 0.254) (layer B.Cu) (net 22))
 (segment (start 161.541 109.22) (end 151.3105 98.9895) (width 0.254) (layer B.Cu) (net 22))
 (segment (start 168.91 109.22) (end 161.541 109.22) (width 0.254) (layer B.Cu) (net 22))
 (segment (start 139.7 90.17) (end 139.7 89.0267) (width 0.254) (layer B.Cu) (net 21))
 (segment (start 172.5956 105.5344) (end 171.45 106.68) (width 0.254) (layer B.Cu) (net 21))
 (segment (start 172.5956 101.1286) (end 172.5956 105.5344) (width 0.254) (layer B.Cu) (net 21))
 (segment (start 160.0138 88.5468) (end 172.5956 101.1286) (width 0.254) (layer B.Cu) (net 21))
 (segment (start 151.4995 88.5468) (end 160.0138 88.5468) (width 0.254) (layer B.Cu) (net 21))
 (segment (start 151.0196 89.0267) (end 151.4995 88.5468) (width 0.254) (layer B.Cu) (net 21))
 (segment (start 139.7 89.0267) (end 151.0196 89.0267) (width 0.254) (layer B.Cu) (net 21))
 (segment (start 151.5431 89.0181) (end 151.8976 89.3726) (width 0.254) (layer F.Cu) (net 18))
 (segment (start 139.2316 89.0181) (end 151.5431 89.0181) (width 0.254) (layer F.Cu) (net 18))
 (segment (start 138.2919 89.9578) (end 139.2316 89.0181) (width 0.254) (layer F.Cu) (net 18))
 (segment (start 138.2919 90.17) (end 138.2919 89.9578) (width 0.254) (layer F.Cu) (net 18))
 (segment (start 155.5393 89.3726) (end 167.7667 101.6) (width 0.254) (layer B.Cu) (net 18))
 (segment (start 151.8976 89.3726) (end 155.5393 89.3726) (width 0.254) (layer B.Cu) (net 18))
 (segment (start 137.16 90.17) (end 138.2919 90.17) (width 0.254) (layer F.Cu) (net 18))
 (segment (start 168.91 101.6) (end 167.7667 101.6) (width 0.254) (layer B.Cu) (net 18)))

